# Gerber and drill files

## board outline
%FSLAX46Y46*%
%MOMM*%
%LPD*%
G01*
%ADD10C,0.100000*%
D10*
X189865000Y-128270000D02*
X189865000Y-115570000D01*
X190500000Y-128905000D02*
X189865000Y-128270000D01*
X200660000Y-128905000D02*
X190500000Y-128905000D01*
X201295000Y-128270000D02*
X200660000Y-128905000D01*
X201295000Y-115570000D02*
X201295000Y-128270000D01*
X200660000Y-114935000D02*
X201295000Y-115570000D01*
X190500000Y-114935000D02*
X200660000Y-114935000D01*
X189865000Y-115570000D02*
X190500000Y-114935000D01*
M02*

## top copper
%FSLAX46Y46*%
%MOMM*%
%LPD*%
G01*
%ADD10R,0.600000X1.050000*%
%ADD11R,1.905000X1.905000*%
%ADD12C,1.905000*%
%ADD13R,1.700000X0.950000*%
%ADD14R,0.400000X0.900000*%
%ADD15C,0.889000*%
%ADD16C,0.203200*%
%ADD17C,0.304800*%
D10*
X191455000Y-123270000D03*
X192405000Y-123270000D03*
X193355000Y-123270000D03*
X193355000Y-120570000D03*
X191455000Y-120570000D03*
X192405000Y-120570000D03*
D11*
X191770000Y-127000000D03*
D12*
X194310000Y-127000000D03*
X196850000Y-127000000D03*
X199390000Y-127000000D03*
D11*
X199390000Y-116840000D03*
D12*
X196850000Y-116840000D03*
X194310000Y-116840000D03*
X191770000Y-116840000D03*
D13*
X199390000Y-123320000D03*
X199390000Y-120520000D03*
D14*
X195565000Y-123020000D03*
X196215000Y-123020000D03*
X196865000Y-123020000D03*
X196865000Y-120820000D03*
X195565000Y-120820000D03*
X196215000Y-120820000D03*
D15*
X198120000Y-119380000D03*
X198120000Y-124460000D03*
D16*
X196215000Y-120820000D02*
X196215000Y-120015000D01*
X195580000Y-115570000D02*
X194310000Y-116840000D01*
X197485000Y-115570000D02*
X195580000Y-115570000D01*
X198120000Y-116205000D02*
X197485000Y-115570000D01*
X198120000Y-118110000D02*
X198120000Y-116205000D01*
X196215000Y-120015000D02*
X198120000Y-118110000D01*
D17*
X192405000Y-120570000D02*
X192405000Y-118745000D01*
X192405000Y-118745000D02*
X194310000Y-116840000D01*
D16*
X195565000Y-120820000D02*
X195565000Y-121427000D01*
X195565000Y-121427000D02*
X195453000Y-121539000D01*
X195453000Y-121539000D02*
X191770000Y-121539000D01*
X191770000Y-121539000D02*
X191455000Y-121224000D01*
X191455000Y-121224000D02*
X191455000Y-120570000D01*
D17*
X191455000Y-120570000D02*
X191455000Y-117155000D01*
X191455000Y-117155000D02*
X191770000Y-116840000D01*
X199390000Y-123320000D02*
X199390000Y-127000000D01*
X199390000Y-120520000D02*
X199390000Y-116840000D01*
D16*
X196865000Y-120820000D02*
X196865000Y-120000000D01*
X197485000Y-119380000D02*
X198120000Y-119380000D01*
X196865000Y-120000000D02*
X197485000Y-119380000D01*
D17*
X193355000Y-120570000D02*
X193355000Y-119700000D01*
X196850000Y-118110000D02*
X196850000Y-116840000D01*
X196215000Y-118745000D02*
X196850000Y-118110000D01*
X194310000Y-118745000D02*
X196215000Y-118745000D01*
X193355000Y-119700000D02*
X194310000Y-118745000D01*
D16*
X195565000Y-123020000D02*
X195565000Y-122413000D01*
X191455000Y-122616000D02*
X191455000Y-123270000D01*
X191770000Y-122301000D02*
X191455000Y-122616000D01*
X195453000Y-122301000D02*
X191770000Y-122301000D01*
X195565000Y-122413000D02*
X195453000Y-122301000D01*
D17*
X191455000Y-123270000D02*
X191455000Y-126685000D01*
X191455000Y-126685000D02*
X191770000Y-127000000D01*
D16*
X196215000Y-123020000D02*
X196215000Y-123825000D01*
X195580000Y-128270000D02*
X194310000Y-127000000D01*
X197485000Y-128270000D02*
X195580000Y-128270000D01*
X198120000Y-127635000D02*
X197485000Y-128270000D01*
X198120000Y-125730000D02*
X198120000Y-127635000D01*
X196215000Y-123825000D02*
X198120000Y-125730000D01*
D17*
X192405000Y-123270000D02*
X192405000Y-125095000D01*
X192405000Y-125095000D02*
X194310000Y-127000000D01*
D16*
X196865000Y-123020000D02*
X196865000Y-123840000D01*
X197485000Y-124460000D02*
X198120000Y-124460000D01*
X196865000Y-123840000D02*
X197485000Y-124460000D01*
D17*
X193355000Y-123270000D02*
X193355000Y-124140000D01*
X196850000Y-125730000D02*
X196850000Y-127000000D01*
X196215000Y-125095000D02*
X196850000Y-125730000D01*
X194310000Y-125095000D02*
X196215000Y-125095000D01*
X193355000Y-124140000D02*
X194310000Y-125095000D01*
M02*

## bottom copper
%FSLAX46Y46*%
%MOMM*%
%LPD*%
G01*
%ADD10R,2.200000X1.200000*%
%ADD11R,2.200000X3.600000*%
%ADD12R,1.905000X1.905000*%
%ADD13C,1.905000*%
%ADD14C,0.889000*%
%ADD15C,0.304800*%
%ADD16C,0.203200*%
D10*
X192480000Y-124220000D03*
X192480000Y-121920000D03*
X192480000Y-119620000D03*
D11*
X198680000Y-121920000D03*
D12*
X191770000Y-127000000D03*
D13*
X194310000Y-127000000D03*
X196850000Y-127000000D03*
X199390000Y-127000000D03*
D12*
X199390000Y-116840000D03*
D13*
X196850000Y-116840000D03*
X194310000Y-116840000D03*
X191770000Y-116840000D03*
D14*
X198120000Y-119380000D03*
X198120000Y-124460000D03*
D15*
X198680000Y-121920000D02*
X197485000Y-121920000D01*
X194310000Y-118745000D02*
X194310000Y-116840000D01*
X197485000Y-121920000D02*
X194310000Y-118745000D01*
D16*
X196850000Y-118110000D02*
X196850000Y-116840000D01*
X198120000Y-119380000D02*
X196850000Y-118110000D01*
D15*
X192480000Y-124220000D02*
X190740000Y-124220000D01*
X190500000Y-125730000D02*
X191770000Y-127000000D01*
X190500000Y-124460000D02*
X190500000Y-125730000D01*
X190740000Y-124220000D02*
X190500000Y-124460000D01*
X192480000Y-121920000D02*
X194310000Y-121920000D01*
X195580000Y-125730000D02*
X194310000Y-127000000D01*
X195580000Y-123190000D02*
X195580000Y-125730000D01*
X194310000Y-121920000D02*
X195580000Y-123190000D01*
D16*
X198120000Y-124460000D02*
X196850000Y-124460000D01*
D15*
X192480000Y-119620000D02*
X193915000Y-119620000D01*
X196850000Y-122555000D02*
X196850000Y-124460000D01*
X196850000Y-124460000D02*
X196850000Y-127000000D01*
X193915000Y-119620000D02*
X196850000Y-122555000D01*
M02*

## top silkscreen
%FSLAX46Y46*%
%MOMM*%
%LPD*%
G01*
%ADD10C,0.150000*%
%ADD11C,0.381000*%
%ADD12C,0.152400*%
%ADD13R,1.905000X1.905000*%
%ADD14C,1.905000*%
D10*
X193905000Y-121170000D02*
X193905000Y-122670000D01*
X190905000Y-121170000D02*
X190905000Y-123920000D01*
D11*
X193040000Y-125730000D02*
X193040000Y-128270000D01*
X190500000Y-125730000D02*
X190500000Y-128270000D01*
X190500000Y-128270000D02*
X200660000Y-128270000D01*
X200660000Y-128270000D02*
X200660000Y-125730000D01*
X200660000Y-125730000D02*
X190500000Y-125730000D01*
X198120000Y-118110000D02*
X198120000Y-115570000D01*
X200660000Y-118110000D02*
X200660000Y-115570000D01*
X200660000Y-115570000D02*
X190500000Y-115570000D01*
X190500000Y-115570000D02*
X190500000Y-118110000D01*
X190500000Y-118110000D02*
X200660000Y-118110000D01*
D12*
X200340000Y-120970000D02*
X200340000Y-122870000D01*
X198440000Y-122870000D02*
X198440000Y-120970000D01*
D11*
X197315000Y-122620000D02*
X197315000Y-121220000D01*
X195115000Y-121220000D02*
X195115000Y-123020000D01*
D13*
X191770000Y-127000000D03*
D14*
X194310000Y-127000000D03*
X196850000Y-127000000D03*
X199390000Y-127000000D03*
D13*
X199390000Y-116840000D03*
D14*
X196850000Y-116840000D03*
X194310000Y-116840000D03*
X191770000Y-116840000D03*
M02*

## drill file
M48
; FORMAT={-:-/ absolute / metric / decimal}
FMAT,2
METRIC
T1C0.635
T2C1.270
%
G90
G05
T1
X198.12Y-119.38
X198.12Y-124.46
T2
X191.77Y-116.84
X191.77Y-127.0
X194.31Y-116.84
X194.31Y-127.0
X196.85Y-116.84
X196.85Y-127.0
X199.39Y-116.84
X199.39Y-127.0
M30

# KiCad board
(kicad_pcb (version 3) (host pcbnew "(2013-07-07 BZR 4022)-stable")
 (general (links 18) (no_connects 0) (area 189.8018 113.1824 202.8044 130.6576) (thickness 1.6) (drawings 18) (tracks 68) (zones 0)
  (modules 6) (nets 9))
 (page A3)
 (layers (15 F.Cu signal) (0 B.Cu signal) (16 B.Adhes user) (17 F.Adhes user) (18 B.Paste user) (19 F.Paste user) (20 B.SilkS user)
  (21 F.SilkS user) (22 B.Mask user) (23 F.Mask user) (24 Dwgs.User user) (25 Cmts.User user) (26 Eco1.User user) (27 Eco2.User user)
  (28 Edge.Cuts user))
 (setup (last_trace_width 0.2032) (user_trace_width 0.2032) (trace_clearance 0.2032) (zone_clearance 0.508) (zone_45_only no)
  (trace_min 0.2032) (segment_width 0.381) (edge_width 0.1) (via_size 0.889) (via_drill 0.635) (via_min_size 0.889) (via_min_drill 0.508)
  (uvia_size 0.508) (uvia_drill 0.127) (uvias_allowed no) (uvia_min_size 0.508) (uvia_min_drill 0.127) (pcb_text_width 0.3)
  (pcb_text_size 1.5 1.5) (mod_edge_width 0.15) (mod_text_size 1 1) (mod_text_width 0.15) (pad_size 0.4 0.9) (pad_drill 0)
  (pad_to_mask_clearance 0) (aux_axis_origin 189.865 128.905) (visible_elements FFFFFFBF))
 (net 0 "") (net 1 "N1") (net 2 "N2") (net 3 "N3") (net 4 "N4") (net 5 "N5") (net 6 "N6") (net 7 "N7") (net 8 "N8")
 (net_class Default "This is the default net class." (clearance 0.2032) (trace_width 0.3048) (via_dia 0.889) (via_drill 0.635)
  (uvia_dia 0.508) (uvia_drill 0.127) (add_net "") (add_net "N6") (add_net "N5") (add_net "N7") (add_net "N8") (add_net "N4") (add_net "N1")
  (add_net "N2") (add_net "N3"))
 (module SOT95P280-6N (layer F.Cu) (at 192.405 121.92)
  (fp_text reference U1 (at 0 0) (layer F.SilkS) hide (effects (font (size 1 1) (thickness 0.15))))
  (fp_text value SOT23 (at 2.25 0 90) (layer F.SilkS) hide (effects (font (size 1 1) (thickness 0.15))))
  (fp_line (start 1.5 -0.75) (end 1.5 0.75) (layer F.SilkS) (width 0.15))
  (fp_line (start -1.5 -0.75) (end -1.5 2) (layer F.SilkS) (width 0.15))
  (pad 1 smd rect (at -0.95 1.35) (size 0.6 1.05) (layers F.Cu F.Paste F.Mask) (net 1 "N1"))
  (pad 2 smd rect (at 0 1.35) (size 0.6 1.05) (layers F.Cu F.Paste F.Mask) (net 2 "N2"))
  (pad 3 smd rect (at 0.95 1.35) (size 0.6 1.05) (layers F.Cu F.Paste F.Mask) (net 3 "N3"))
  (pad 4 smd rect (at 0.95 -1.35) (size 0.6 1.05) (layers F.Cu F.Paste F.Mask) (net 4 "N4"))
  (pad 6 smd rect (at -0.95 -1.35) (size 0.6 1.05) (layers F.Cu F.Paste F.Mask) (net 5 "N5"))
  (pad 5 smd rect (at 0 -1.35) (size 0.6 1.05) (layers F.Cu F.Paste F.Mask) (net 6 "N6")))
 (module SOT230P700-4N (layer B.Cu) (at 195.58 121.92 90)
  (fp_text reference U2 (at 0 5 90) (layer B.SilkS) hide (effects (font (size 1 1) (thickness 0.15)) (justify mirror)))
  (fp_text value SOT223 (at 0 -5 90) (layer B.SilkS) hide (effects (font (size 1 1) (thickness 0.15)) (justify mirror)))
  (pad 1 smd rect (at -2.3 -3.1 90) (size 1.2 2.2) (layers B.Cu B.Paste B.Mask) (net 1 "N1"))
  (pad 2 smd rect (at 0 -3.1 90) (size 1.2 2.2) (layers B.Cu B.Paste B.Mask) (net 2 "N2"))
  (pad 3 smd rect (at 2.3 -3.1 90) (size 1.2 2.2) (layers B.Cu B.Paste B.Mask) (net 3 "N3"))
  (pad 4 smd rect (at 0 3.1 90) (size 3.6 2.2) (layers B.Cu B.Paste B.Mask) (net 6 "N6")))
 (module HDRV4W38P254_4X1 (layer F.Cu) (at 195.58 127)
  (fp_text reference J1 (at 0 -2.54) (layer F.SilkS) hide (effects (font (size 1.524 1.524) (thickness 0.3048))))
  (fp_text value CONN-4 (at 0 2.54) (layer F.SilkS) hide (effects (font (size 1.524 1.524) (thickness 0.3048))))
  (fp_line (start -2.54 -1.27) (end -2.54 1.27) (layer F.SilkS) (width 0.381))
  (fp_line (start -5.08 -1.27) (end -5.08 1.27) (layer F.SilkS) (width 0.381))
  (fp_line (start -5.08 1.27) (end 5.08 1.27) (layer F.SilkS) (width 0.381))
  (fp_line (start 5.08 1.27) (end 5.08 -1.27) (layer F.SilkS) (width 0.381))
  (fp_line (start 5.08 -1.27) (end -5.08 -1.27) (layer F.SilkS) (width 0.381))
  (pad 1 thru_hole rect (at -3.81 0) (size 1.905 1.905) (drill 1.27) (layers *.Cu *.Mask F.SilkS) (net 1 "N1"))
  (pad 2 thru_hole circle (at -1.27 0) (size 1.905 1.905) (drill 1.27) (layers *.Cu *.Mask F.SilkS) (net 2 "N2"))
  (pad 3 thru_hole circle (at 1.27 0) (size 1.905 1.905) (drill 1.27) (layers *.Cu *.Mask F.SilkS) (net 3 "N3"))
  (pad 4 thru_hole circle (at 3.81 0) (size 1.905 1.905) (drill 1.27) (layers *.Cu *.Mask F.SilkS) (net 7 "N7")))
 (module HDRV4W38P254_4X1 (layer F.Cu) (at 195.58 116.84 180)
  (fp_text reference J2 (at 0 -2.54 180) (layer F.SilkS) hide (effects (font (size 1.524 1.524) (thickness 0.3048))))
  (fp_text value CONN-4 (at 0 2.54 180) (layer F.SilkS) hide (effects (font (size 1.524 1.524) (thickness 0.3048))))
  (fp_line (start -2.54 -1.27) (end -2.54 1.27) (layer F.SilkS) (width 0.381))
  (fp_line (start -5.08 -1.27) (end -5.08 1.27) (layer F.SilkS) (width 0.381))
  (fp_line (start -5.08 1.27) (end 5.08 1.27) (layer F.SilkS) (width 0.381))
  (fp_line (start 5.08 1.27) (end 5.08 -1.27) (layer F.SilkS) (width 0.381))
  (fp_line (start 5.08 -1.27) (end -5.08 -1.27) (layer F.SilkS) (width 0.381))
  (pad 1 thru_hole rect (at -3.81 0 180) (size 1.905 1.905) (drill 1.27) (layers *.Cu *.Mask F.SilkS) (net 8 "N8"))
  (pad 2 thru_hole circle (at -1.27 0 180) (size 1.905 1.905) (drill 1.27) (layers *.Cu *.Mask F.SilkS) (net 4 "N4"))
  (pad 3 thru_hole circle (at 1.27 0 180) (size 1.905 1.905) (drill 1.27) (layers *.Cu *.Mask F.SilkS) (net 6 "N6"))
  (pad 4 thru_hole circle (at 3.81 0 180) (size 1.905 1.905) (drill 1.27) (layers *.Cu *.Mask F.SilkS) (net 5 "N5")))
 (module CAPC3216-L (layer F.Cu) (at 199.39 121.92 90)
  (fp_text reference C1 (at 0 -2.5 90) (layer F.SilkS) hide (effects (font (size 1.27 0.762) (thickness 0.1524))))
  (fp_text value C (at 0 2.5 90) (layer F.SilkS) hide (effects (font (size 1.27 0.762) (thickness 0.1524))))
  (fp_line (start 0.95 0.95) (end -0.95 0.95) (layer F.SilkS) (width 0.1524))
  (fp_line (start -0.95 -0.95) (end 0.95 -0.95) (layer F.SilkS) (width 0.1524))
  (pad 1 smd rect (at -1.4 0 90) (size 0.95 1.7) (layers F.Cu F.Paste F.Mask) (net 7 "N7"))
  (pad 2 smd rect (at 1.4 0 90) (size 0.95 1.7) (layers F.Cu F.Paste F.Mask) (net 8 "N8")))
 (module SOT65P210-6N (layer F.Cu) (at 196.215 121.92)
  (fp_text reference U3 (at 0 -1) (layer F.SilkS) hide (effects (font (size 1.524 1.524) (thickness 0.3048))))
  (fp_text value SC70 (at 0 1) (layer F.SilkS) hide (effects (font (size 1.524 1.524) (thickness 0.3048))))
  (fp_line (start 1.1 0.7) (end 1.1 -0.7) (layer F.SilkS) (width 0.381))
  (fp_line (start -1.1 -0.7) (end -1.1 1.1) (layer F.SilkS) (width 0.381))
  (pad 1 smd rect (at -0.65 1.1) (size 0.4 0.9) (layers F.Cu F.Paste F.Mask) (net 1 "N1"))
  (pad 2 smd rect (at 0 1.1) (size 0.4 0.9) (layers F.Cu F.Paste F.Mask) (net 2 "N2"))
  (pad 3 smd rect (at 0.65 1.1) (size 0.4 0.9) (layers F.Cu F.Paste F.Mask) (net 3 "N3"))
  (pad 4 smd rect (at 0.65 -1.1) (size 0.4 0.9) (layers F.Cu F.Paste F.Mask) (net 4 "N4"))
  (pad 6 smd rect (at -0.65 -1.1) (size 0.4 0.9) (layers F.Cu F.Paste F.Mask) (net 5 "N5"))
  (pad 5 smd rect (at 0 -1.1) (size 0.4 0.9) (layers F.Cu F.Paste F.Mask) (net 6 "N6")))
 (gr_line (start 189.865 128.27) (end 189.865 115.57) (angle 90) (layer Edge.Cuts) (width 0.1))
 (gr_line (start 190.5 128.905) (end 189.865 128.27) (angle 90) (layer Edge.Cuts) (width 0.1))
 (gr_line (start 200.66 128.905) (end 190.5 128.905) (angle 90) (layer Edge.Cuts) (width 0.1))
 (gr_line (start 201.295 128.27) (end 200.66 128.905) (angle 90) (layer Edge.Cuts) (width 0.1))
 (gr_line (start 201.295 115.57) (end 201.295 128.27) (angle 90) (layer Edge.Cuts) (width 0.1))
 (gr_line (start 200.66 114.935) (end 201.295 115.57) (angle 90) (layer Edge.Cuts) (width 0.1))
 (gr_line (start 190.5 114.935) (end 200.66 114.935) (angle 90) (layer Edge.Cuts) (width 0.1))
 (gr_line (start 189.865 115.57) (end 190.5 114.935) (angle 90) (layer Edge.Cuts) (width 0.1))
 (segment (start 196.215 120.82) (end 196.215 120.015) (width 0.2032) (layer F.Cu) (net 6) (status 400000))
 (segment (start 195.58 115.57) (end 194.31 116.84) (width 0.2032) (layer F.Cu) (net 6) (status 800000))
 (segment (start 197.485 115.57) (end 195.58 115.57) (width 0.2032) (layer F.Cu) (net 6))
 (segment (start 198.12 116.205) (end 197.485 115.57) (width 0.2032) (layer F.Cu) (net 6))
 (segment (start 198.12 118.11) (end 198.12 116.205) (width 0.2032) (layer F.Cu) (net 6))
 (segment (start 196.215 120.015) (end 198.12 118.11) (width 0.2032) (layer F.Cu) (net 6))
 (segment (start 192.405 120.57) (end 192.405 118.745) (width 0.3048) (layer F.Cu) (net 6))
 (segment (start 192.405 118.745) (end 194.31 116.84) (width 0.3048) (layer F.Cu) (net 6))
 (segment (start 198.68 121.92) (end 197.485 121.92) (width 0.3048) (layer B.Cu) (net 6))
 (segment (start 194.31 118.745) (end 194.31 116.84) (width 0.3048) (layer B.Cu) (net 6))
 (segment (start 197.485 121.92) (end 194.31 118.745) (width 0.3048) (layer B.Cu) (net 6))
 (segment (start 195.565 120.82) (end 195.565 121.427) (width 0.2032) (layer F.Cu) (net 5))
 (segment (start 195.565 121.427) (end 195.453 121.539) (width 0.2032) (layer F.Cu) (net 5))
 (segment (start 195.453 121.539) (end 191.77 121.539) (width 0.2032) (layer F.Cu) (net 5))
 (segment (start 191.77 121.539) (end 191.455 121.224) (width 0.2032) (layer F.Cu) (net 5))
 (segment (start 191.455 121.224) (end 191.455 120.57) (width 0.2032) (layer F.Cu) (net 5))
 (segment (start 191.455 120.57) (end 191.455 117.155) (width 0.3048) (layer F.Cu) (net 5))
 (segment (start 191.455 117.155) (end 191.77 116.84) (width 0.3048) (layer F.Cu) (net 5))
 (segment (start 199.39 123.32) (end 199.39 127) (width 0.3048) (layer F.Cu) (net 7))
 (segment (start 199.39 120.52) (end 199.39 116.84) (width 0.3048) (layer F.Cu) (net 8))
 (segment (start 196.865 120.82) (end 196.865 120) (width 0.2032) (layer F.Cu) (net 4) (status 400000))
 (segment (start 196.85 118.11) (end 196.85 116.84) (width 0.2032) (layer B.Cu) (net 4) (status 800000))
 (segment (start 198.12 119.38) (end 196.85 118.11) (width 0.2032) (layer B.Cu) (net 4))
 (via (at 198.12 119.38) (size 0.889) (layers F.Cu B.Cu) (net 4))
 (segment (start 197.485 119.38) (end 198.12 119.38) (width 0.2032) (layer F.Cu) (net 4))
 (segment (start 196.865 120) (end 197.485 119.38) (width 0.2032) (layer F.Cu) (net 4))
 (segment (start 193.355 120.57) (end 193.355 119.7) (width 0.3048) (layer F.Cu) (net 4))
 (segment (start 196.85 118.11) (end 196.85 116.84) (width 0.3048) (layer F.Cu) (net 4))
 (segment (start 196.215 118.745) (end 196.85 118.11) (width 0.3048) (layer F.Cu) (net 4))
 (segment (start 194.31 118.745) (end 196.215 118.745) (width 0.3048) (layer F.Cu) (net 4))
 (segment (start 193.355 119.7) (end 194.31 118.745) (width 0.3048) (layer F.Cu) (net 4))
 (segment (start 195.565 123.02) (end 195.565 122.413) (width 0.2032) (layer F.Cu) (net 1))
 (segment (start 191.455 122.616) (end 191.455 123.27) (width 0.2032) (layer F.Cu) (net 1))
 (segment (start 191.77 122.301) (end 191.455 122.616) (width 0.2032) (layer F.Cu) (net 1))
 (segment (start 195.453 122.301) (end 191.77 122.301) (width 0.2032) (layer F.Cu) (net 1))
 (segment (start 195.565 122.413) (end 195.453 122.301) (width 0.2032) (layer F.Cu) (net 1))
 (segment (start 191.455 123.27) (end 191.455 126.685) (width 0.3048) (layer F.Cu) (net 1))
 (segment (start 191.455 126.685) (end 191.77 127) (width 0.3048) (layer F.Cu) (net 1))
 (segment (start 192.48 124.22) (end 190.74 124.22) (width 0.3048) (layer B.Cu) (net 1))
 (segment (start 190.5 125.73) (end 191.77 127) (width 0.3048) (layer B.Cu) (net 1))
 (segment (start 190.5 124.46) (end 190.5 125.73) (width 0.3048) (layer B.Cu) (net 1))
 (segment (start 190.74 124.22) (end 190.5 124.46) (width 0.3048) (layer B.Cu) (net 1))
 (segment (start 196.215 123.02) (end 196.215 123.825) (width 0.2032) (layer F.Cu) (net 2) (status 400000))
 (segment (start 195.58 128.27) (end 194.31 127) (width 0.2032) (layer F.Cu) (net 2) (status 800000))
 (segment (start 197.485 128.27) (end 195.58 128.27) (width 0.2032) (layer F.Cu) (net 2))
 (segment (start 198.12 127.635) (end 197.485 128.27) (width 0.2032) (layer F.Cu) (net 2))
 (segment (start 198.12 125.73) (end 198.12 127.635) (width 0.2032) (layer F.Cu) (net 2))
 (segment (start 196.215 123.825) (end 198.12 125.73) (width 0.2032) (layer F.Cu) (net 2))
 (segment (start 192.405 123.27) (end 192.405 125.095) (width 0.3048) (layer F.Cu) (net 2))
 (segment (start 192.405 125.095) (end 194.31 127) (width 0.3048) (layer F.Cu) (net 2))
 (segment (start 192.48 121.92) (end 194.31 121.92) (width 0.3048) (layer B.Cu) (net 2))
 (segment (start 195.58 125.73) (end 194.31 127) (width 0.3048) (layer B.Cu) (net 2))
 (segment (start 195.58 123.19) (end 195.58 125.73) (width 0.3048) (layer B.Cu) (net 2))
 (segment (start 194.31 121.92) (end 195.58 123.19) (width 0.3048) (layer B.Cu) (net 2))
 (segment (start 196.865 123.02) (end 196.865 123.84) (width 0.2032) (layer F.Cu) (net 3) (status 400000))
 (segment (start 198.12 124.46) (end 196.85 124.46) (width 0.2032) (layer B.Cu) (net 3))
 (via (at 198.12 124.46) (size 0.889) (layers F.Cu B.Cu) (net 3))
 (segment (start 197.485 124.46) (end 198.12 124.46) (width 0.2032) (layer F.Cu) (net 3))
 (segment (start 196.865 123.84) (end 197.485 124.46) (width 0.2032) (layer F.Cu) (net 3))
 (segment (start 193.355 123.27) (end 193.355 124.14) (width 0.3048) (layer F.Cu) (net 3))
 (segment (start 196.85 125.73) (end 196.85 127) (width 0.3048) (layer F.Cu) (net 3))
 (segment (start 196.215 125.095) (end 196.85 125.73) (width 0.3048) (layer F.Cu) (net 3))
 (segment (start 194.31 125.095) (end 196.215 125.095) (width 0.3048) (layer F.Cu) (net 3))
 (segment (start 193.355 124.14) (end 194.31 125.095) (width 0.3048) (layer F.Cu) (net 3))
 (segment (start 192.48 119.62) (end 193.915 119.62) (width 0.3048) (layer B.Cu) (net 3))
 (segment (start 196.85 122.555) (end 196.85 124.46) (width 0.3048) (layer B.Cu) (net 3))
 (segment (start 196.85 124.46) (end 196.85 127) (width 0.3048) (layer B.Cu) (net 3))
 (segment (start 193.915 119.62) (end 196.85 122.555) (width 0.3048) (layer B.Cu) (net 3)))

